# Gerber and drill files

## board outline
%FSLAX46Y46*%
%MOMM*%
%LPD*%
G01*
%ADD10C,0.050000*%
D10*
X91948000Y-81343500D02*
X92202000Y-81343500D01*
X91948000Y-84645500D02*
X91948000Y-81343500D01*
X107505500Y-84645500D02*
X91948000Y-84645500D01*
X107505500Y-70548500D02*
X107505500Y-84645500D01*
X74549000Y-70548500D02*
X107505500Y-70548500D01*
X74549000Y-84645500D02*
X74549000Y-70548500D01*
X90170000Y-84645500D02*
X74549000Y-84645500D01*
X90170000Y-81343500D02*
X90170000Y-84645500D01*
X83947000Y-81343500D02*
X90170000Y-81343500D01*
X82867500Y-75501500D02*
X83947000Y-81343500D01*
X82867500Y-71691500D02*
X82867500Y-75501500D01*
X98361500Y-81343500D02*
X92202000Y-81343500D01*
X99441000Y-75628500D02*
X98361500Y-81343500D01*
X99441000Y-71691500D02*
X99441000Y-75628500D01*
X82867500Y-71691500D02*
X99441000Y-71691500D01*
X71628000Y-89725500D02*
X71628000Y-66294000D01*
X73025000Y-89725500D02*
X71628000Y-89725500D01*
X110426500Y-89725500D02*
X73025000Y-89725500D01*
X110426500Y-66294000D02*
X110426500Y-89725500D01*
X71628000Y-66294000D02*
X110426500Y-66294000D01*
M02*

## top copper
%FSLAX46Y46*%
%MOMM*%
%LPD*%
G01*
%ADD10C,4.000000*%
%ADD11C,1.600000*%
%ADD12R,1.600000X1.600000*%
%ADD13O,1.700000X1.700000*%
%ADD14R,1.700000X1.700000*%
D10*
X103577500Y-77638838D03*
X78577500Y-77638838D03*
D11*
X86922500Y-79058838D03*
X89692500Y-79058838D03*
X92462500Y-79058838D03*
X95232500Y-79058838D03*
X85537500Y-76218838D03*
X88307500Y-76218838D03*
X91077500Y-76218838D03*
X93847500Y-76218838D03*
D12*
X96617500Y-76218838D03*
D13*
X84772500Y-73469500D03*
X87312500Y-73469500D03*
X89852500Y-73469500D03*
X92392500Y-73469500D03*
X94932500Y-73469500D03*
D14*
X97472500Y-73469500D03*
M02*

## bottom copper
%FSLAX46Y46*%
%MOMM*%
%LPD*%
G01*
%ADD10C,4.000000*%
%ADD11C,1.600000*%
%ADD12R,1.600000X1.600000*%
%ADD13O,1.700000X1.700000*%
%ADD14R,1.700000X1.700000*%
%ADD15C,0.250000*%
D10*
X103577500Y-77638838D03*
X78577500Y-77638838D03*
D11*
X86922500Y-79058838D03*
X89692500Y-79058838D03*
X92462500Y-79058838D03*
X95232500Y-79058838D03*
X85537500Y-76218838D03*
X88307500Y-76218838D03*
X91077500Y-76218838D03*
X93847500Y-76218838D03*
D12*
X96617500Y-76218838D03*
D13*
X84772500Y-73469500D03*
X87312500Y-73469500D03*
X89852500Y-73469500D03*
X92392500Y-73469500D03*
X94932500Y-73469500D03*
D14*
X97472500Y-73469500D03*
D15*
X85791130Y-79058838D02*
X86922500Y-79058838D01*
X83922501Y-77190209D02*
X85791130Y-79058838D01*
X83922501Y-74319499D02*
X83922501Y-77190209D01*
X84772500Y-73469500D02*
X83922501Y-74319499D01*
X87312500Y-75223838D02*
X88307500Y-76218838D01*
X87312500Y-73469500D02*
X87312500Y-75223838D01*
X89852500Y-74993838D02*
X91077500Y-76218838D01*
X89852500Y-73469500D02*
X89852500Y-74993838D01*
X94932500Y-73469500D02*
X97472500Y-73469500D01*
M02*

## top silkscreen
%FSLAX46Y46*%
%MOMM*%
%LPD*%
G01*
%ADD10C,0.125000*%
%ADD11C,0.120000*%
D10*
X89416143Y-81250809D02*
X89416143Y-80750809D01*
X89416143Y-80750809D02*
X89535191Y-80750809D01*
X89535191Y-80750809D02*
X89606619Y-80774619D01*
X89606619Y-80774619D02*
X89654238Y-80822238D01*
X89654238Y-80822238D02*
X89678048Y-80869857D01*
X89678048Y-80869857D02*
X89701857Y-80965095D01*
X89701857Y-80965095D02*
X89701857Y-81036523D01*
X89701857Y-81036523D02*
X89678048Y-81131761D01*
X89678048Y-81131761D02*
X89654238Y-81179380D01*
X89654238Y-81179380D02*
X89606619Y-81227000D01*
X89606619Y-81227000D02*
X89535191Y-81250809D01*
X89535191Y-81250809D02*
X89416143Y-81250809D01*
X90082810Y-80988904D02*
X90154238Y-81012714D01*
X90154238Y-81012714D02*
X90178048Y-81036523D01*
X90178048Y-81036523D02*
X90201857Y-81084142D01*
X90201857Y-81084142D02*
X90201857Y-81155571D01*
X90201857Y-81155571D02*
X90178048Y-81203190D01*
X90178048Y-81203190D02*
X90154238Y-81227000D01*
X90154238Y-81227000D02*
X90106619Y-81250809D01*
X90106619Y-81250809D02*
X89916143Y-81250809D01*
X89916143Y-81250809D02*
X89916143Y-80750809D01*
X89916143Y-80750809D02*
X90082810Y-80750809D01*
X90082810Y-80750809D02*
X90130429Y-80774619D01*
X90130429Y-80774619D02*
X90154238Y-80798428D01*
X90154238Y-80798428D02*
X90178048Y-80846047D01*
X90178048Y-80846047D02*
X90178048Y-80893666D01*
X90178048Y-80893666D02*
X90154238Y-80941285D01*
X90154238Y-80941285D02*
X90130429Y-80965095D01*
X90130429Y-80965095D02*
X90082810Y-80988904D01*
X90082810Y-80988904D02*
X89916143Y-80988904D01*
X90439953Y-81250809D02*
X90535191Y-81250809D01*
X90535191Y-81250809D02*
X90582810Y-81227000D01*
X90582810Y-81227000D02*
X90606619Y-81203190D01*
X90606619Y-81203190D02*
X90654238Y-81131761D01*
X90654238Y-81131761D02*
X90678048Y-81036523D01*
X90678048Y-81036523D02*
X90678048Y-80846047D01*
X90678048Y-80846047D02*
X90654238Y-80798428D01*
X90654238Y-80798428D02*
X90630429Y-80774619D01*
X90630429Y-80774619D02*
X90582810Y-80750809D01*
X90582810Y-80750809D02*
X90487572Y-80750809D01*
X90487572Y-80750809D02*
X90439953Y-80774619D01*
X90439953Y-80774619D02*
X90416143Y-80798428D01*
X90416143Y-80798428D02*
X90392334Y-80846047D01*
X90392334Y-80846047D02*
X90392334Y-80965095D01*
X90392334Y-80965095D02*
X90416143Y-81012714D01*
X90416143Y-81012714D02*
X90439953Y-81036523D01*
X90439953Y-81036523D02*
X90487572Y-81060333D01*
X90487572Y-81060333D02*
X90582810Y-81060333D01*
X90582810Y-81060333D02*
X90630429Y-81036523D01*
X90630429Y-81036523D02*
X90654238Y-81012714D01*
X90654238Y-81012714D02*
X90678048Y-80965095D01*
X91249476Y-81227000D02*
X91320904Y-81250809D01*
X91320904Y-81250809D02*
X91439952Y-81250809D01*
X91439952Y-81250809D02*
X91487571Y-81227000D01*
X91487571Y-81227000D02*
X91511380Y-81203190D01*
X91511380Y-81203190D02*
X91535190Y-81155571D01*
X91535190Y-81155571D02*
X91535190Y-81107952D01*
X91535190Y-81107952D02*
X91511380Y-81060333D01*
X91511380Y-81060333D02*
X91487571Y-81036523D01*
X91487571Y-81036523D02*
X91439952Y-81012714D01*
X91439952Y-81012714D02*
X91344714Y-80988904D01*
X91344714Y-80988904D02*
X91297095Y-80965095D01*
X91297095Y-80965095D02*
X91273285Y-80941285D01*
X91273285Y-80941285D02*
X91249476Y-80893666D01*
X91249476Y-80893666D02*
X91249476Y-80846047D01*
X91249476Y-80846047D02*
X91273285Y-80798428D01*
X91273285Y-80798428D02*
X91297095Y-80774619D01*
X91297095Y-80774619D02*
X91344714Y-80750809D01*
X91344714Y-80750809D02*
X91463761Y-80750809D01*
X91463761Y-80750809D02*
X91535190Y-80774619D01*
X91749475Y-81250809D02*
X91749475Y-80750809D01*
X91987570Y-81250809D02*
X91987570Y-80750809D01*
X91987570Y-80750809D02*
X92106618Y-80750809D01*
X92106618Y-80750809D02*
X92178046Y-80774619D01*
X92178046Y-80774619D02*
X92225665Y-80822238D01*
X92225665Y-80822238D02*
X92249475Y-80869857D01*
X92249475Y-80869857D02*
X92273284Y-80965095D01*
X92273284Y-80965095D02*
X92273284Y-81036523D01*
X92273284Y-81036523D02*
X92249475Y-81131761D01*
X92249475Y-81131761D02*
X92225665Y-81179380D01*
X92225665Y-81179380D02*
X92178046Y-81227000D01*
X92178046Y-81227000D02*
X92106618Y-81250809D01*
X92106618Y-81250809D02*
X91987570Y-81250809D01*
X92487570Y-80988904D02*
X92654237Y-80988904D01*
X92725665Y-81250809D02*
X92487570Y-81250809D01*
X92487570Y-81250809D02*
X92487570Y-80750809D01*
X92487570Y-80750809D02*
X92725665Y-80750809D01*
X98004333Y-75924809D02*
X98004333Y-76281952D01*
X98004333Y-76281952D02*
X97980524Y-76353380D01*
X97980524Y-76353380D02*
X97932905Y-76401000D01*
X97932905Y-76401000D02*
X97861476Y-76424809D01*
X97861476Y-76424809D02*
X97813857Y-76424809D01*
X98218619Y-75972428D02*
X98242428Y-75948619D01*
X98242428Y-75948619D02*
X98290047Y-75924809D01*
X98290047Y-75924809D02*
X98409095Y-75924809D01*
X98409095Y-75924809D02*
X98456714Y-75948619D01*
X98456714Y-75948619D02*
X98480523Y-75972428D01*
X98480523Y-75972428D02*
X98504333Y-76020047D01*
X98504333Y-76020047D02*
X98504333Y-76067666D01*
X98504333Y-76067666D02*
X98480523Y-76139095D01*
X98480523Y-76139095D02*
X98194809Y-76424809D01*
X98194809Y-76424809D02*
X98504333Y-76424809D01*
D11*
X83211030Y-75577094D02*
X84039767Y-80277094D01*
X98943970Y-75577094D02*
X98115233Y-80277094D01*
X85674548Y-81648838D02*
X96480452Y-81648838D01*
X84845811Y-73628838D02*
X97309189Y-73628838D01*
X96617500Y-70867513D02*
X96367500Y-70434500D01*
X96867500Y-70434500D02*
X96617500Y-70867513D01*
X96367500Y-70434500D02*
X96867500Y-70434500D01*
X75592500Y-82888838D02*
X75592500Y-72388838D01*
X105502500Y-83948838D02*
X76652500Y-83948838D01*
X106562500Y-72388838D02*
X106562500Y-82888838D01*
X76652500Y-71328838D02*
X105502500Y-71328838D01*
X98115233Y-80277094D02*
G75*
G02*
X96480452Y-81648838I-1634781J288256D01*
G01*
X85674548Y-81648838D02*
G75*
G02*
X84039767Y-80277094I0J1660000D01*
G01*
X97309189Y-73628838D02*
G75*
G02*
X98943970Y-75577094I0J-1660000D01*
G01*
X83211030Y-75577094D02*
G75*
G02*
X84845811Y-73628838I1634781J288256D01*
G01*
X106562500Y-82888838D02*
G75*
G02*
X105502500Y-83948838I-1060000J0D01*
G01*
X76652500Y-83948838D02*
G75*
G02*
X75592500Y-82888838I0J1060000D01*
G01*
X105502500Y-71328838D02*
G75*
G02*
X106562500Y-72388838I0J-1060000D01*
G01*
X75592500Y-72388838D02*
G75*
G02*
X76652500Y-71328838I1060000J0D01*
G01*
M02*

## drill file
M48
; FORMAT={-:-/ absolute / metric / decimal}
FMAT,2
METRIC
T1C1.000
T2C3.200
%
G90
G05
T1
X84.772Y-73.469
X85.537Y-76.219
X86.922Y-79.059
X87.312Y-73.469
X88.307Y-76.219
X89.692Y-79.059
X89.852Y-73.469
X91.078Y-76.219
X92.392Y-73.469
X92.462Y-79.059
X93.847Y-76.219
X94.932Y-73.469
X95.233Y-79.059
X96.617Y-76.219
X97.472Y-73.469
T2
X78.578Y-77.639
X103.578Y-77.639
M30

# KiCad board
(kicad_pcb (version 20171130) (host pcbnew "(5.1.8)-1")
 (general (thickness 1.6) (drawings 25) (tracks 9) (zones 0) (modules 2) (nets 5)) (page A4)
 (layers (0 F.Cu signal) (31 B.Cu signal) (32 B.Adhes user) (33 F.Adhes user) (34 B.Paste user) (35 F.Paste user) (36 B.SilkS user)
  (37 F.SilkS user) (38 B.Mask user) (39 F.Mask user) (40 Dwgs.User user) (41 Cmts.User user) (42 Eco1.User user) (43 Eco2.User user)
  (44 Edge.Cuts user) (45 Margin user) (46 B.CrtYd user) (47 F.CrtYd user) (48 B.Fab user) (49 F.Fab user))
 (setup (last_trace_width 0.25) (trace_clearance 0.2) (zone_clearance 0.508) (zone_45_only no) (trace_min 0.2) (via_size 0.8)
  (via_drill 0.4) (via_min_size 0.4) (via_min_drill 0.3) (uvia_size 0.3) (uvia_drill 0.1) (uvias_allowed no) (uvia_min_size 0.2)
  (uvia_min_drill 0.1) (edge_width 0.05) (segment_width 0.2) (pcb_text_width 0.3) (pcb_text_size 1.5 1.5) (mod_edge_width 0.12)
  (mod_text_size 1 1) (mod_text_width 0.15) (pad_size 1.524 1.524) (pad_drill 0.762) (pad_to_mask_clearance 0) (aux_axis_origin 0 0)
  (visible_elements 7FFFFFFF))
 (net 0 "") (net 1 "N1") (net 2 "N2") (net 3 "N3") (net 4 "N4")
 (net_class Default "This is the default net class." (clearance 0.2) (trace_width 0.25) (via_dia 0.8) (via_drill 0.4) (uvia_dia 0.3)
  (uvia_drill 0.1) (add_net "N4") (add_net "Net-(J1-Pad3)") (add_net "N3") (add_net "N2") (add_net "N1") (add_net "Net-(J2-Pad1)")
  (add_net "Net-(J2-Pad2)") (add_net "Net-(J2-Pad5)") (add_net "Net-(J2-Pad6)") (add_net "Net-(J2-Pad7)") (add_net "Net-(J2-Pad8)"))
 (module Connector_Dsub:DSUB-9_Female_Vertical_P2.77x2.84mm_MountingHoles (layer F.Cu) (at 96.6175 76.218838)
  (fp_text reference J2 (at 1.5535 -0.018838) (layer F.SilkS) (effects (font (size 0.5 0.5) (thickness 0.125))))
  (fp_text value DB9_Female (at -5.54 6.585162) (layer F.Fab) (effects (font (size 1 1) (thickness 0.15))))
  (fp_line (start -13.40647 -0.641744) (end -12.577733 4.058256) (layer F.SilkS) (width 0.12))
  (fp_line (start 2.32647 -0.641744) (end 1.497733 4.058256) (layer F.SilkS) (width 0.12))
  (fp_line (start -10.942952 5.43) (end -0.137048 5.43) (layer F.SilkS) (width 0.12))
  (fp_line (start -11.771689 -2.59) (end 0.691689 -2.59) (layer F.SilkS) (width 0.12))
  (fp_line (start 0 -5.351325) (end -0.25 -5.784338) (layer F.SilkS) (width 0.12))
  (fp_line (start 0.25 -5.784338) (end 0 -5.351325) (layer F.SilkS) (width 0.12))
  (fp_line (start -0.25 -5.784338) (end 0.25 -5.784338) (layer F.SilkS) (width 0.12))
  (fp_line (start -21.025 6.67) (end -21.025 -3.83) (layer F.SilkS) (width 0.12))
  (fp_line (start 8.885 7.73) (end -19.965 7.73) (layer F.SilkS) (width 0.12))
  (fp_line (start 9.945 -3.83) (end 9.945 6.67) (layer F.SilkS) (width 0.12))
  (fp_line (start -19.965 -4.89) (end 8.885 -4.89) (layer F.SilkS) (width 0.12))
  (fp_arc (start -0.137048 3.77) (end -0.137048 5.43) (angle -80) (layer F.SilkS) (width 0.12))
  (fp_arc (start -10.942952 3.77) (end -10.942952 5.43) (angle 80) (layer F.SilkS) (width 0.12))
  (fp_arc (start 0.691689 -0.93) (end 0.691689 -2.59) (angle 100) (layer F.SilkS) (width 0.12))
  (fp_arc (start -11.771689 -0.93) (end -11.771689 -2.59) (angle -100) (layer F.SilkS) (width 0.12))
  (fp_arc (start 8.885 6.67) (end 9.945 6.67) (angle 90) (layer F.SilkS) (width 0.12))
  (fp_arc (start -19.965 6.67) (end -21.025 6.67) (angle -90) (layer F.SilkS) (width 0.12))
  (fp_arc (start 8.885 -3.83) (end 8.885 -4.89) (angle 90) (layer F.SilkS) (width 0.12))
  (fp_arc (start -19.965 -3.83) (end -21.025 -3.83) (angle 90) (layer F.SilkS) (width 0.12))
  (pad 0 thru_hole circle (at 6.96 1.42) (size 4 4) (drill 3.2) (layers *.Cu *.Mask))
  (pad 0 thru_hole circle (at -18.04 1.42) (size 4 4) (drill 3.2) (layers *.Cu *.Mask))
  (pad 9 thru_hole circle (at -9.695 2.84) (size 1.6 1.6) (drill 1) (layers *.Cu *.Mask) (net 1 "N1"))
  (pad 8 thru_hole circle (at -6.925 2.84) (size 1.6 1.6) (drill 1) (layers *.Cu *.Mask))
  (pad 7 thru_hole circle (at -4.155 2.84) (size 1.6 1.6) (drill 1) (layers *.Cu *.Mask))
  (pad 6 thru_hole circle (at -1.385 2.84) (size 1.6 1.6) (drill 1) (layers *.Cu *.Mask))
  (pad 5 thru_hole circle (at -11.08 0) (size 1.6 1.6) (drill 1) (layers *.Cu *.Mask))
  (pad 4 thru_hole circle (at -8.31 0) (size 1.6 1.6) (drill 1) (layers *.Cu *.Mask) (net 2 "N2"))
  (pad 3 thru_hole circle (at -5.54 0) (size 1.6 1.6) (drill 1) (layers *.Cu *.Mask) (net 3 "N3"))
  (pad 2 thru_hole circle (at -2.77 0) (size 1.6 1.6) (drill 1) (layers *.Cu *.Mask))
  (pad 1 thru_hole rect (at 0 0) (size 1.6 1.6) (drill 1) (layers *.Cu *.Mask)))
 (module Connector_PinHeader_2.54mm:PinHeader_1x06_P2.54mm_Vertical (layer B.Cu) (at 97.4725 73.4695 90)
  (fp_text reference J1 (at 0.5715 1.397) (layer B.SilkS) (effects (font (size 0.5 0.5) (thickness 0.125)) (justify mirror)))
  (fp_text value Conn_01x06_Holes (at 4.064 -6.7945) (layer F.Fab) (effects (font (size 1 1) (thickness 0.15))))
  (pad 6 thru_hole oval (at 0 -12.7 90) (size 1.7 1.7) (drill 1) (layers *.Cu *.Mask) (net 1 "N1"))
  (pad 5 thru_hole oval (at 0 -10.16 90) (size 1.7 1.7) (drill 1) (layers *.Cu *.Mask) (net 2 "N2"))
  (pad 4 thru_hole oval (at 0 -7.62 90) (size 1.7 1.7) (drill 1) (layers *.Cu *.Mask) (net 3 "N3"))
  (pad 3 thru_hole oval (at 0 -5.08 90) (size 1.7 1.7) (drill 1) (layers *.Cu *.Mask))
  (pad 2 thru_hole oval (at 0 -2.54 90) (size 1.7 1.7) (drill 1) (layers *.Cu *.Mask) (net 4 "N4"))
  (pad 1 thru_hole rect (at 0 0 90) (size 1.7 1.7) (drill 1) (layers *.Cu *.Mask) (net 4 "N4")))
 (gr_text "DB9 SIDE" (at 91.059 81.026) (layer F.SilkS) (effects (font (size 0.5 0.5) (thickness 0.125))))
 (gr_line (start 91.948 81.3435) (end 92.202 81.3435) (layer Edge.Cuts) (width 0.05))
 (gr_line (start 91.948 84.6455) (end 91.948 81.3435) (layer Edge.Cuts) (width 0.05))
 (gr_line (start 107.5055 84.6455) (end 91.948 84.6455) (layer Edge.Cuts) (width 0.05))
 (gr_line (start 107.5055 70.5485) (end 107.5055 84.6455) (layer Edge.Cuts) (width 0.05))
 (gr_line (start 74.549 70.5485) (end 107.5055 70.5485) (layer Edge.Cuts) (width 0.05))
 (gr_line (start 74.549 84.6455) (end 74.549 70.5485) (layer Edge.Cuts) (width 0.05))
 (gr_line (start 90.17 84.6455) (end 74.549 84.6455) (layer Edge.Cuts) (width 0.05))
 (gr_line (start 90.17 81.3435) (end 90.17 84.6455) (layer Edge.Cuts) (width 0.05))
 (gr_line (start 83.947 81.3435) (end 90.17 81.3435) (layer Edge.Cuts) (width 0.05))
 (gr_line (start 82.8675 75.5015) (end 83.947 81.3435) (layer Edge.Cuts) (width 0.05))
 (gr_line (start 82.8675 71.6915) (end 82.8675 75.5015) (layer Edge.Cuts) (width 0.05))
 (gr_line (start 98.3615 81.3435) (end 92.202 81.3435) (layer Edge.Cuts) (width 0.05))
 (gr_line (start 99.441 75.6285) (end 98.3615 81.3435) (layer Edge.Cuts) (width 0.05))
 (gr_line (start 99.441 71.6915) (end 99.441 75.6285) (layer Edge.Cuts) (width 0.05))
 (gr_line (start 82.8675 71.6915) (end 99.441 71.6915) (layer Edge.Cuts) (width 0.05))
 (gr_line (start 71.628 89.7255) (end 71.628 66.294) (layer Edge.Cuts) (width 0.05))
 (gr_line (start 73.025 89.7255) (end 71.628 89.7255) (layer Edge.Cuts) (width 0.05))
 (gr_line (start 110.4265 89.7255) (end 73.025 89.7255) (layer Edge.Cuts) (width 0.05))
 (gr_line (start 110.4265 66.294) (end 110.4265 89.7255) (layer Edge.Cuts) (width 0.05))
 (gr_line (start 71.628 66.294) (end 110.4265 66.294) (layer Edge.Cuts) (width 0.05))
 (segment (start 85.79113 79.058838) (end 86.9225 79.058838) (width 0.25) (layer B.Cu) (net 1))
 (segment (start 83.922501 77.190209) (end 85.79113 79.058838) (width 0.25) (layer B.Cu) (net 1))
 (segment (start 83.922501 74.319499) (end 83.922501 77.190209) (width 0.25) (layer B.Cu) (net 1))
 (segment (start 84.7725 73.4695) (end 83.922501 74.319499) (width 0.25) (layer B.Cu) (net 1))
 (segment (start 87.3125 75.223838) (end 88.3075 76.218838) (width 0.25) (layer B.Cu) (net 2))
 (segment (start 87.3125 73.4695) (end 87.3125 75.223838) (width 0.25) (layer B.Cu) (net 2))
 (segment (start 89.8525 74.993838) (end 91.0775 76.218838) (width 0.25) (layer B.Cu) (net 3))
 (segment (start 89.8525 73.4695) (end 89.8525 74.993838) (width 0.25) (layer B.Cu) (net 3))
 (segment (start 94.9325 73.4695) (end 97.4725 73.4695) (width 0.25) (layer B.Cu) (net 4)))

